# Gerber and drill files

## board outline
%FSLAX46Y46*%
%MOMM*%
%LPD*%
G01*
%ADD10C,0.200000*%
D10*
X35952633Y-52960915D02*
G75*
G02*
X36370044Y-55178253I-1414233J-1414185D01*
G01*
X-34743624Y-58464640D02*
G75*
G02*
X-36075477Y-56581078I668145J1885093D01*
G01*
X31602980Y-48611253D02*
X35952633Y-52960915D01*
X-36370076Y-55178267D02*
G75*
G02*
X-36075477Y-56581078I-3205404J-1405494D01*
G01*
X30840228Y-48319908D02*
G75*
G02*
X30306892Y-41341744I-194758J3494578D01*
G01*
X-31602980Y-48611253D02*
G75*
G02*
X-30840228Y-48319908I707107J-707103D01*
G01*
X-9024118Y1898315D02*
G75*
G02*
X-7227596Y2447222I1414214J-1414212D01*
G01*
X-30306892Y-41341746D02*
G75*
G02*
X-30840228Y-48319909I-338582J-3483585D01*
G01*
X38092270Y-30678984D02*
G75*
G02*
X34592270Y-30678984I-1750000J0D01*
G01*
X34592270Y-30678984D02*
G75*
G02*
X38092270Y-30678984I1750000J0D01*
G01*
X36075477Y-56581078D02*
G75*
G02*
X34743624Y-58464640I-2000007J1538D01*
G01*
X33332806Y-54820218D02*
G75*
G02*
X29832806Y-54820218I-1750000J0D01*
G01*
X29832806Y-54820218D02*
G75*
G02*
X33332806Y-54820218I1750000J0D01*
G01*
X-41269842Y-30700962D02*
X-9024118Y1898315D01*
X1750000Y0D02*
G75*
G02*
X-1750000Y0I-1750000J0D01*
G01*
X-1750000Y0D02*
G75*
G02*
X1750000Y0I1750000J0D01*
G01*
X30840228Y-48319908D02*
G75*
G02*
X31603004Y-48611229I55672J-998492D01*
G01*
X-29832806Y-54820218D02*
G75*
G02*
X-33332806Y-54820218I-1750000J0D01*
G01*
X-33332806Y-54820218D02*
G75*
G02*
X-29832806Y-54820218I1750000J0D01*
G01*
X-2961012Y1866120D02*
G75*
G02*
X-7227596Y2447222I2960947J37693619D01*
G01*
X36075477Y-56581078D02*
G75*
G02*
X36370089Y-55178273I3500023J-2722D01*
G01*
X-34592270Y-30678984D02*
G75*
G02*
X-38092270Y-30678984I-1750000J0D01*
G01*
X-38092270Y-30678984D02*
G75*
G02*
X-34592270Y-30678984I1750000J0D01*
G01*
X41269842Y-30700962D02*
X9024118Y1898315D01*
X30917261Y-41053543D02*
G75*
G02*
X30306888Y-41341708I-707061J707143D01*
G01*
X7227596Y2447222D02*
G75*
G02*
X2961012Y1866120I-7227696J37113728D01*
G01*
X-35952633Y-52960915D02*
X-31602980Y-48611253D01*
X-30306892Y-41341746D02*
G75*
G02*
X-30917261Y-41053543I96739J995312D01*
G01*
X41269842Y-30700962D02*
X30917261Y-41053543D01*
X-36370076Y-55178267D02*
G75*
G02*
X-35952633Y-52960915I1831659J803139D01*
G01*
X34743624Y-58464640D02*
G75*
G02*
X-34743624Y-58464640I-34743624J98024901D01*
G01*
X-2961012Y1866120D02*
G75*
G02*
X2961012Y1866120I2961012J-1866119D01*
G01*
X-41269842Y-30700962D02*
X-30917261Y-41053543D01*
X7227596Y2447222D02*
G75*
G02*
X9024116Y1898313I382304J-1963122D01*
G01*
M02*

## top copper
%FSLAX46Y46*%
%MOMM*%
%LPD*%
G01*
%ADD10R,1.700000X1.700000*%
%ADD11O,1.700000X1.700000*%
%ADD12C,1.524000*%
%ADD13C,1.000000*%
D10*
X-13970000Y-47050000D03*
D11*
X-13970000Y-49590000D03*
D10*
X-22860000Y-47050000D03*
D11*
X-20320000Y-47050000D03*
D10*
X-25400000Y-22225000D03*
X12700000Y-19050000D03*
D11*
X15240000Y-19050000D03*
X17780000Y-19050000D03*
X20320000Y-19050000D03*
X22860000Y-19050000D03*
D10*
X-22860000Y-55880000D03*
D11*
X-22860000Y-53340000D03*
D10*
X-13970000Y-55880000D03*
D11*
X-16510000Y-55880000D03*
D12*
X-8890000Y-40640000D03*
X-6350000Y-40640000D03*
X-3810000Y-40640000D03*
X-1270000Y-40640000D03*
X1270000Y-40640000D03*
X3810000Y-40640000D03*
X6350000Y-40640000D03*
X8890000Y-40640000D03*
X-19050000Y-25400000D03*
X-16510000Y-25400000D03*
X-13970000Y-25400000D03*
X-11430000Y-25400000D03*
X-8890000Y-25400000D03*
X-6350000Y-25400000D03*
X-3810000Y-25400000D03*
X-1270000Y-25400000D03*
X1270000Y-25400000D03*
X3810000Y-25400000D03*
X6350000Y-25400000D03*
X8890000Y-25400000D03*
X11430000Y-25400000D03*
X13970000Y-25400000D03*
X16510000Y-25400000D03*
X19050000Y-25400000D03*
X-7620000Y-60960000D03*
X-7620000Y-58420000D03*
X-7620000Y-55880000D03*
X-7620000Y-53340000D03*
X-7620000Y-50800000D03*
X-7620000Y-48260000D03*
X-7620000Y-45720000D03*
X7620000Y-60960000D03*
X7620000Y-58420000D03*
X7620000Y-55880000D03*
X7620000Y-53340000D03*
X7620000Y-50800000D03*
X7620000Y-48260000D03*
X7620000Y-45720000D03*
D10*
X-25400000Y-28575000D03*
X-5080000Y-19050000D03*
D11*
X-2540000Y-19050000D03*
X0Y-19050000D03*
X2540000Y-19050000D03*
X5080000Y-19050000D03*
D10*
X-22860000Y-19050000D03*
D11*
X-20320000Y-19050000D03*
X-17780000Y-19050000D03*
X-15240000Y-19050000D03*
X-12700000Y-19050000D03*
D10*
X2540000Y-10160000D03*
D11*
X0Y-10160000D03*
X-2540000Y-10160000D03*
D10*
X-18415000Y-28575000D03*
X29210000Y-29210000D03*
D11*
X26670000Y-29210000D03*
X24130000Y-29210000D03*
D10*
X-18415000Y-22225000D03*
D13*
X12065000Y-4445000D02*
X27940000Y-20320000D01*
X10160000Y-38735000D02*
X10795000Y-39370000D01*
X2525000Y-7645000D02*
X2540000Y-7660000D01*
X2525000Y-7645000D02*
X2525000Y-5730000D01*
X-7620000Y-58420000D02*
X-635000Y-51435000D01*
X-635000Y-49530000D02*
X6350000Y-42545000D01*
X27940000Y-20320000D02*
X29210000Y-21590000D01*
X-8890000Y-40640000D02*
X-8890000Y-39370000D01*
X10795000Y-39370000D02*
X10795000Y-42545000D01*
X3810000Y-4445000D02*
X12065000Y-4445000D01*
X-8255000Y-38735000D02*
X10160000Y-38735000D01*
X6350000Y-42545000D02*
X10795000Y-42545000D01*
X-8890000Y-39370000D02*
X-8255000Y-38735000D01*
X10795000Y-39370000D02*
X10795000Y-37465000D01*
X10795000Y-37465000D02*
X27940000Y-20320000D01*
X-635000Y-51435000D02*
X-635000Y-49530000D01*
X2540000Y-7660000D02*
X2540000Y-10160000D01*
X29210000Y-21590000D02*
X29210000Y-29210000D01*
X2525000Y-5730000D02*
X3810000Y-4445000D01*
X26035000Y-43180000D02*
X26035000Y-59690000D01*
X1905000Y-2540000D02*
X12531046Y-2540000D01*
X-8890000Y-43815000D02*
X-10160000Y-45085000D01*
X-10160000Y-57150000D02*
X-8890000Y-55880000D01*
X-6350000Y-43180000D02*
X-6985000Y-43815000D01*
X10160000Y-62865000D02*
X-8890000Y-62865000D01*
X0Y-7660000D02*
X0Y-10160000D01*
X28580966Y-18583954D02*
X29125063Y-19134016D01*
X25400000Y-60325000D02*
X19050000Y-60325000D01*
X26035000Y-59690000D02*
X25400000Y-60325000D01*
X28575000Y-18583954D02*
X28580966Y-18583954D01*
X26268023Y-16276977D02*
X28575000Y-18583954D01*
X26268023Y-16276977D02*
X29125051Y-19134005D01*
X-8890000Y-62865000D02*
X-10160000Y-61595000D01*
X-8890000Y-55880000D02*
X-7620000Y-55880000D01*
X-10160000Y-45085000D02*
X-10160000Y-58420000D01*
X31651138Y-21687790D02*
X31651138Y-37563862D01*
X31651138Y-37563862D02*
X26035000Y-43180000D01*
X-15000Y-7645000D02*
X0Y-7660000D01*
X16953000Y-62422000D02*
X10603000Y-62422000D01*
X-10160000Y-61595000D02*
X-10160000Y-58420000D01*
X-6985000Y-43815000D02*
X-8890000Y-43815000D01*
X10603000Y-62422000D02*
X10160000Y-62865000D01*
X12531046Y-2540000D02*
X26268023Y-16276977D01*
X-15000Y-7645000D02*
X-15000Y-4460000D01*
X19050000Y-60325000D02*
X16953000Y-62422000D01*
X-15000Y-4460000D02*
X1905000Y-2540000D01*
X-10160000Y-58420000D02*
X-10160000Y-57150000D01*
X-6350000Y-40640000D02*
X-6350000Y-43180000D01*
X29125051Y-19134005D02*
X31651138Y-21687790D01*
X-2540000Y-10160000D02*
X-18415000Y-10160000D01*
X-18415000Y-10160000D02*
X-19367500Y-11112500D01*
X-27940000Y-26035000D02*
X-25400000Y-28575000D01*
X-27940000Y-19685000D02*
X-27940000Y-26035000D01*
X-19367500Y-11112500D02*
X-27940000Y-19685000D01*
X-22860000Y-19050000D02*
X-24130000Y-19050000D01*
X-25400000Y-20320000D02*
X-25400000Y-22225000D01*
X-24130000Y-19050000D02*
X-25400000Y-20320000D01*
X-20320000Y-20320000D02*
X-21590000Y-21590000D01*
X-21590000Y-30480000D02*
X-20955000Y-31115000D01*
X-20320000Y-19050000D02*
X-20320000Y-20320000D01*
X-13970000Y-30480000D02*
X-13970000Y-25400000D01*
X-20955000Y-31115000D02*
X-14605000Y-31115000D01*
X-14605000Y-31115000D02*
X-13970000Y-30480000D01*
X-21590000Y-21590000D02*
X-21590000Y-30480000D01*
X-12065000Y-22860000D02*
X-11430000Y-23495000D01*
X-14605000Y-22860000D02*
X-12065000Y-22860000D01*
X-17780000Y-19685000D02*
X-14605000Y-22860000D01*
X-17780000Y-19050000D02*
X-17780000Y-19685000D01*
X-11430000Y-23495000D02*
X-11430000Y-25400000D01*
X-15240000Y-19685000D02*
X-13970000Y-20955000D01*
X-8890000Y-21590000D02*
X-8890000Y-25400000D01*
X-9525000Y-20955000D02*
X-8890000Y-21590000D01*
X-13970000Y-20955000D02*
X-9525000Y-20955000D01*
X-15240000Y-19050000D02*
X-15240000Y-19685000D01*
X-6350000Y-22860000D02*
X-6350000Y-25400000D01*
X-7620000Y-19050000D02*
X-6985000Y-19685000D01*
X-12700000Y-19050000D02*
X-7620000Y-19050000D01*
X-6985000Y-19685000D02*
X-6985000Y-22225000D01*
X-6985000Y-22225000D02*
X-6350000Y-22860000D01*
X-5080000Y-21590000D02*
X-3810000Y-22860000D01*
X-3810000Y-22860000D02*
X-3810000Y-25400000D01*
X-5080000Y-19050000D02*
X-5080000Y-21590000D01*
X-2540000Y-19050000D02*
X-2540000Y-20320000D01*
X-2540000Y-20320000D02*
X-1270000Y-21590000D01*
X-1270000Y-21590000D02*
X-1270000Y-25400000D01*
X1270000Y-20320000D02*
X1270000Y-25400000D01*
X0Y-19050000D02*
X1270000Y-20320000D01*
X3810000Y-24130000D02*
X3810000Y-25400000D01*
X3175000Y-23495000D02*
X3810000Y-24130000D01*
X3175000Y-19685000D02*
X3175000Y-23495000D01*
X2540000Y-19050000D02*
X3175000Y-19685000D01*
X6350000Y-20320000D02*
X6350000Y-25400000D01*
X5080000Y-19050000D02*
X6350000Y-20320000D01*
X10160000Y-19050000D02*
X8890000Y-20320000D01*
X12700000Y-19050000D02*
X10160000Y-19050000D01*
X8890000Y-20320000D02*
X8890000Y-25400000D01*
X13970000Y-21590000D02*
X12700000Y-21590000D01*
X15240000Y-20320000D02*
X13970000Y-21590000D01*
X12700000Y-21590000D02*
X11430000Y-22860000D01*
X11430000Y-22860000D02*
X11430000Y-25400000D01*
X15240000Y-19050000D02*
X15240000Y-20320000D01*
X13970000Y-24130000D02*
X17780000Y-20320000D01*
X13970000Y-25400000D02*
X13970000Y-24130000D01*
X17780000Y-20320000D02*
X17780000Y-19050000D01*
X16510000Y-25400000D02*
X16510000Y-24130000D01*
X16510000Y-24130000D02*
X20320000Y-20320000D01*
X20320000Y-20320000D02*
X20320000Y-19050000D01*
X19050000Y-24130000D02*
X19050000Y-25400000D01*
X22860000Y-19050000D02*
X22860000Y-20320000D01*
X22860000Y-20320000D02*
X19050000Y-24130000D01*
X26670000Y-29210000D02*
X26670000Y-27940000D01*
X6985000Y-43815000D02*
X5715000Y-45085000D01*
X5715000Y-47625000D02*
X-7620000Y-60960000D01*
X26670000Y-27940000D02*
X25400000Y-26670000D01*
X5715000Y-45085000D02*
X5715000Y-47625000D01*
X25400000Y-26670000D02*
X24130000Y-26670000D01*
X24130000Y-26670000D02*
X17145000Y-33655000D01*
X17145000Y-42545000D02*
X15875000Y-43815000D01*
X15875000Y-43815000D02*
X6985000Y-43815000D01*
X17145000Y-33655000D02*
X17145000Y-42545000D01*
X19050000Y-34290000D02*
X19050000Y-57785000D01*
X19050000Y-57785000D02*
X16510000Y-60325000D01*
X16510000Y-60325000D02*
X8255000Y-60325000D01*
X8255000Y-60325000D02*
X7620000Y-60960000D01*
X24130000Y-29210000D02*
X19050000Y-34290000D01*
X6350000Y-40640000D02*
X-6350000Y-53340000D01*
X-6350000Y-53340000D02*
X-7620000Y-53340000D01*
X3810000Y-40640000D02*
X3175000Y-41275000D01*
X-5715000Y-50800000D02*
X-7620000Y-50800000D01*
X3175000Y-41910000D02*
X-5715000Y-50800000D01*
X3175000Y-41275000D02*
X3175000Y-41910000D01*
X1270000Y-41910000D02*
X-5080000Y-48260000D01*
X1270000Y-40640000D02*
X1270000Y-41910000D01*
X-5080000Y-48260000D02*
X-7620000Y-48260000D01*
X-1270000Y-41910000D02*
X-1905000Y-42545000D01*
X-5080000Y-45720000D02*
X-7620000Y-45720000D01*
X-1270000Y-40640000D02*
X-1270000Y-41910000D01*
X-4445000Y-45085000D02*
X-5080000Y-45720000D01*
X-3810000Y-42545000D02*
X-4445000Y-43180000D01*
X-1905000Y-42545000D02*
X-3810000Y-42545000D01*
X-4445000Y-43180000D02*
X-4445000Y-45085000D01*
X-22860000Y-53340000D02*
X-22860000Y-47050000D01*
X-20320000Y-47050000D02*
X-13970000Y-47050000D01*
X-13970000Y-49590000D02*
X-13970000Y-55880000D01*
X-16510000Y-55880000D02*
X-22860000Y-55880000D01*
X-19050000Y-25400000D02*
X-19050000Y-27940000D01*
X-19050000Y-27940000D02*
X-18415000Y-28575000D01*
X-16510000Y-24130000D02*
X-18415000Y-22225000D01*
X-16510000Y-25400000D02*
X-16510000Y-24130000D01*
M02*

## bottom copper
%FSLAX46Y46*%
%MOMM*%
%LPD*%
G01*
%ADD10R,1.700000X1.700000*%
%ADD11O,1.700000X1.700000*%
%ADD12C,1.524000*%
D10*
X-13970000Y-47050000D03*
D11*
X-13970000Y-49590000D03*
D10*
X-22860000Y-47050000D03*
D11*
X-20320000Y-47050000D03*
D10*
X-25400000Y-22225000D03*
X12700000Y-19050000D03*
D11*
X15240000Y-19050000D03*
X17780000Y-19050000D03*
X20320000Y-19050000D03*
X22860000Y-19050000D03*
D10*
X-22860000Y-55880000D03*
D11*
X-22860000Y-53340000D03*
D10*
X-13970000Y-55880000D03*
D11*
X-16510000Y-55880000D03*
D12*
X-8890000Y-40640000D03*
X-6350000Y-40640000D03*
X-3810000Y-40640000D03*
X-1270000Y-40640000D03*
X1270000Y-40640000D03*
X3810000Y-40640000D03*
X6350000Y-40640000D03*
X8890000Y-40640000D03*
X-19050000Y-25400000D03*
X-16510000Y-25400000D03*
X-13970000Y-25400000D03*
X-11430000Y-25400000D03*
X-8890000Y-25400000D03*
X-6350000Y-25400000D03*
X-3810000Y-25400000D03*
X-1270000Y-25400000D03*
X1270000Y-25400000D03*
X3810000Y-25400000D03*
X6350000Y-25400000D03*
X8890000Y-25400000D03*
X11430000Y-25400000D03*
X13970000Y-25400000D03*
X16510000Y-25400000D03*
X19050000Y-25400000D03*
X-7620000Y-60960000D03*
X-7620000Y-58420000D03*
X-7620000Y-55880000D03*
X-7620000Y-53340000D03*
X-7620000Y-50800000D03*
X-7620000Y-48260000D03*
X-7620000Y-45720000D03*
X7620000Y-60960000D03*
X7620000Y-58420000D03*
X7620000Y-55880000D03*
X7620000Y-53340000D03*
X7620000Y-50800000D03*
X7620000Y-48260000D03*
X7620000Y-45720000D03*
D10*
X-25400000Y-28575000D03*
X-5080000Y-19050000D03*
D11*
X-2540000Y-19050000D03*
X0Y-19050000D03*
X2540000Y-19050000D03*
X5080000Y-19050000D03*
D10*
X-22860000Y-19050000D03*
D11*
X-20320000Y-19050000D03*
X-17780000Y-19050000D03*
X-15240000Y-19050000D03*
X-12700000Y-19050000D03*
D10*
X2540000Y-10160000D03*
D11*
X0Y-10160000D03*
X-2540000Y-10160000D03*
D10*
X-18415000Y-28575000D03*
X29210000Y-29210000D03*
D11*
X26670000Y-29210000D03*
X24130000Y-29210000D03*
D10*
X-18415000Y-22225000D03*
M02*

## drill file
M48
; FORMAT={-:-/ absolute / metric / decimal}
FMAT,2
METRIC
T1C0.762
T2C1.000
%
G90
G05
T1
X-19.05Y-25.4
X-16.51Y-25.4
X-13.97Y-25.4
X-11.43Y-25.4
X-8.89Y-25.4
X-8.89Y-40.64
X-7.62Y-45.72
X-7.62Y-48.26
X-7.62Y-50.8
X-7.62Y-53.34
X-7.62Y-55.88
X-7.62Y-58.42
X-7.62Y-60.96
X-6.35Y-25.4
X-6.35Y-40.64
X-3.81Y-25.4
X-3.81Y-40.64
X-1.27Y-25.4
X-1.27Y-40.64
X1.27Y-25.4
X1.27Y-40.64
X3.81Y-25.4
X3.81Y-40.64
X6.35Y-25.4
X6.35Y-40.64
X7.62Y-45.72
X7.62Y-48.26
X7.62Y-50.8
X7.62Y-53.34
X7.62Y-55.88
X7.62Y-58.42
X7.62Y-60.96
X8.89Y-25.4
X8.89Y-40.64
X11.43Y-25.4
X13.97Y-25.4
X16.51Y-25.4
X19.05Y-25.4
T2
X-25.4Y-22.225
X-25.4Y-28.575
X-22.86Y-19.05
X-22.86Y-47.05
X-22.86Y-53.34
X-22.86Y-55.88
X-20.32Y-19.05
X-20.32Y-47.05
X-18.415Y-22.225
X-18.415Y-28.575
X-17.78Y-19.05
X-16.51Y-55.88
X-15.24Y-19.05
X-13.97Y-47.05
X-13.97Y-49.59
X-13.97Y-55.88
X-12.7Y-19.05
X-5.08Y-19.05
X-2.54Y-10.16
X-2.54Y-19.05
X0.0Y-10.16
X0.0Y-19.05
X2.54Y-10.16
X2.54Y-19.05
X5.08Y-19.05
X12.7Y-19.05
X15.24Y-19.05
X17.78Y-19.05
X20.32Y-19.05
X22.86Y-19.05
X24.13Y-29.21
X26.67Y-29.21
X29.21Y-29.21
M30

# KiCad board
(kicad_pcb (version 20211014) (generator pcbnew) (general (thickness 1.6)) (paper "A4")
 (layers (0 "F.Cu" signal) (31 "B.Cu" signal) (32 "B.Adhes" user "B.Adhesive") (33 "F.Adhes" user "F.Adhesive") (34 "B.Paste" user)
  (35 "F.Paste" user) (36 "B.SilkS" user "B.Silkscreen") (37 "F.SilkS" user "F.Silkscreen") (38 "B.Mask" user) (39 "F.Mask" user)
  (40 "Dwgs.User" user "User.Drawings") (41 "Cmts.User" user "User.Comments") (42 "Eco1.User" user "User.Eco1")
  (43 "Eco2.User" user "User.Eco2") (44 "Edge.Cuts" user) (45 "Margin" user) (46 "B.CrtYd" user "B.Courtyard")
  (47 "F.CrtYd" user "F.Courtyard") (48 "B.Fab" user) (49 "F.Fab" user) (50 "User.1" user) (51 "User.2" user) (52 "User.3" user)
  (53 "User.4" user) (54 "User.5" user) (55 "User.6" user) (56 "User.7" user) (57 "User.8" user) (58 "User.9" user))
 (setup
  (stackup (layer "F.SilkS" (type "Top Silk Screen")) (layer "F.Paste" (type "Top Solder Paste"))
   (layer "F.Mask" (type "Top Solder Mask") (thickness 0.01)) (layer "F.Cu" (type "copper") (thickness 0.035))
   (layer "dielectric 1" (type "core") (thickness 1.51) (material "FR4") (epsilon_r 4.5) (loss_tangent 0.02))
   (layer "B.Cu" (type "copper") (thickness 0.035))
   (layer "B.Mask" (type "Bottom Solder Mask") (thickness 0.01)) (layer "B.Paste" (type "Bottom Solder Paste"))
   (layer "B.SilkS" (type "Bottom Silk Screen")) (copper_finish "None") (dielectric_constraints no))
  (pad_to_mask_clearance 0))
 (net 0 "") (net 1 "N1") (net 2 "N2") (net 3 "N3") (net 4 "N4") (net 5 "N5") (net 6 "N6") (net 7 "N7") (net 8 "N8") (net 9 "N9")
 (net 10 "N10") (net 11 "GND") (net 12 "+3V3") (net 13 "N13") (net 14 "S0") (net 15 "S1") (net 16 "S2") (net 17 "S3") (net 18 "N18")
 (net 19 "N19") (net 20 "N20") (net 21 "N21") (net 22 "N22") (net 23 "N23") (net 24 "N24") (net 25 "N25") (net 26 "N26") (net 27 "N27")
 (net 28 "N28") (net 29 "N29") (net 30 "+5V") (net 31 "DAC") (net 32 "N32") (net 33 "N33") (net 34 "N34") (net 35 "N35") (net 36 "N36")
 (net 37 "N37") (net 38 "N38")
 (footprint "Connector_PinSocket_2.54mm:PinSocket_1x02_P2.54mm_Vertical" (layer "F.Cu") (at -13.97 47.05)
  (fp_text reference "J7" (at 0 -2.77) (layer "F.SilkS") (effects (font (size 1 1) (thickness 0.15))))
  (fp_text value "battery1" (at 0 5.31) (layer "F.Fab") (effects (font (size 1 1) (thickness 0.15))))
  (pad "1" thru_hole rect (at 0 0) (size 1.7 1.7) (drill 1) (layers *.Cu *.Mask) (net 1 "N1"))
  (pad "2" thru_hole oval (at 0 2.54) (size 1.7 1.7) (drill 1) (layers *.Cu *.Mask) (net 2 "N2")))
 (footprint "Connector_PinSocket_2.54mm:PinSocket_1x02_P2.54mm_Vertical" (layer "F.Cu") (at -22.86 47.05 90)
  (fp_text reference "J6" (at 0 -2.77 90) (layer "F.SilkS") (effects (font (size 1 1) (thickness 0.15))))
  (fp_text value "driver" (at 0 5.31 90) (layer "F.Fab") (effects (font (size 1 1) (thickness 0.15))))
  (pad "1" thru_hole rect (at 0 0 90) (size 1.7 1.7) (drill 1) (layers *.Cu *.Mask) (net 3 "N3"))
  (pad "2" thru_hole oval (at 0 2.54 90) (size 1.7 1.7) (drill 1) (layers *.Cu *.Mask) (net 1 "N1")))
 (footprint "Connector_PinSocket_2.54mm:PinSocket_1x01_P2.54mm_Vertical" (layer "F.Cu") (at -25.4 22.225)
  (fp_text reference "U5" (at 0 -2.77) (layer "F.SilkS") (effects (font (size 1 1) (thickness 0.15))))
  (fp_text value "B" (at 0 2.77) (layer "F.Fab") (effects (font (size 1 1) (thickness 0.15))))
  (pad "1" thru_hole rect (at 0 0) (size 1.7 1.7) (drill 1) (layers *.Cu *.Mask) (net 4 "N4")))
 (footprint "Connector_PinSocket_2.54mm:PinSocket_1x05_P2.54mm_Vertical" (layer "F.Cu") (at 12.7 19.05 90)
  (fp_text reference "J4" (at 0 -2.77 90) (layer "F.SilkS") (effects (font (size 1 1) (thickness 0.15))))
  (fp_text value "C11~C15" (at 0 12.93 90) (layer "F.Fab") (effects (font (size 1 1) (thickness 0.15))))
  (pad "1" thru_hole rect (at 0 0 90) (size 1.7 1.7) (drill 1) (layers *.Cu *.Mask) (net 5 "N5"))
  (pad "2" thru_hole oval (at 0 2.54 90) (size 1.7 1.7) (drill 1) (layers *.Cu *.Mask) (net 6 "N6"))
  (pad "3" thru_hole oval (at 0 5.08 90) (size 1.7 1.7) (drill 1) (layers *.Cu *.Mask) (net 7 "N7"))
  (pad "4" thru_hole oval (at 0 7.62 90) (size 1.7 1.7) (drill 1) (layers *.Cu *.Mask) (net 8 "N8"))
  (pad "5" thru_hole oval (at 0 10.16 90) (size 1.7 1.7) (drill 1) (layers *.Cu *.Mask) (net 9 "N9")))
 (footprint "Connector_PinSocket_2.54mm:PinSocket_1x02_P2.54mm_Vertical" (layer "F.Cu") (at -22.86 55.88 180)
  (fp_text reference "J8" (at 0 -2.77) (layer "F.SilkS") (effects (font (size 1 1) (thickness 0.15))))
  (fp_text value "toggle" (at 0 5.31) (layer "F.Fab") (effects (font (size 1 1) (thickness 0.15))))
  (pad "1" thru_hole rect (at 0 0 180) (size 1.7 1.7) (drill 1) (layers *.Cu *.Mask) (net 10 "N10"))
  (pad "2" thru_hole oval (at 0 2.54 180) (size 1.7 1.7) (drill 1) (layers *.Cu *.Mask) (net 3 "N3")))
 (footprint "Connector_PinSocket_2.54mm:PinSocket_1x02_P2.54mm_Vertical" (layer "F.Cu") (at -13.97 55.88 -90)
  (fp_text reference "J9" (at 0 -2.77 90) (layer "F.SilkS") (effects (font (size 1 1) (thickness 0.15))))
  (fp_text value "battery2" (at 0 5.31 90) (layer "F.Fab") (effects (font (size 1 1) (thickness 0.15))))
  (pad "1" thru_hole rect (at 0 0 270) (size 1.7 1.7) (drill 1) (layers *.Cu *.Mask) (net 2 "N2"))
  (pad "2" thru_hole oval (at 0 2.54 270) (size 1.7 1.7) (drill 1) (layers *.Cu *.Mask) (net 10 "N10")))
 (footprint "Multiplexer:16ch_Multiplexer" (layer "F.Cu") (at -1.27 25.4)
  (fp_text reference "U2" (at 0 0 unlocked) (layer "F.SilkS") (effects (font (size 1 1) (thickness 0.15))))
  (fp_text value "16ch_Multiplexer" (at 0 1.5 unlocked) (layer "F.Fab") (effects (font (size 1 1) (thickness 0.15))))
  (pad "1" thru_hole circle (at -7.62 15.24) (size 1.524 1.524) (drill 0.762) (layers *.Cu *.Mask) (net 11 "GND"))
  (pad "2" thru_hole circle (at -5.08 15.24) (size 1.524 1.524) (drill 0.762) (layers *.Cu *.Mask) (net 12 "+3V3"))
  (pad "3" thru_hole circle (at -2.54 15.24) (size 1.524 1.524) (drill 0.762) (layers *.Cu *.Mask) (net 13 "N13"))
  (pad "4" thru_hole circle (at 0 15.24) (size 1.524 1.524) (drill 0.762) (layers *.Cu *.Mask) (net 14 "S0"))
  (pad "5" thru_hole circle (at 2.54 15.24) (size 1.524 1.524) (drill 0.762) (layers *.Cu *.Mask) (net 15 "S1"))
  (pad "6" thru_hole circle (at 5.08 15.24) (size 1.524 1.524) (drill 0.762) (layers *.Cu *.Mask) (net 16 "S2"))
  (pad "7" thru_hole circle (at 7.62 15.24) (size 1.524 1.524) (drill 0.762) (layers *.Cu *.Mask) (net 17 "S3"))
  (pad "8" thru_hole circle (at 10.16 15.24) (size 1.524 1.524) (drill 0.762) (layers *.Cu *.Mask) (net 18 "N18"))
  (pad "9" thru_hole circle (at -17.78 0) (size 1.524 1.524) (drill 0.762) (layers *.Cu *.Mask) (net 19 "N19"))
  (pad "10" thru_hole circle (at -15.24 0) (size 1.524 1.524) (drill 0.762) (layers *.Cu *.Mask) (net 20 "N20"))
  (pad "11" thru_hole circle (at -12.7 0) (size 1.524 1.524) (drill 0.762) (layers *.Cu *.Mask) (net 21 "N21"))
  (pad "12" thru_hole circle (at -10.16 0) (size 1.524 1.524) (drill 0.762) (layers *.Cu *.Mask) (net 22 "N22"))
  (pad "13" thru_hole circle (at -7.62 0) (size 1.524 1.524) (drill 0.762) (layers *.Cu *.Mask) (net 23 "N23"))
  (pad "14" thru_hole circle (at -5.08 0) (size 1.524 1.524) (drill 0.762) (layers *.Cu *.Mask) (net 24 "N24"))
  (pad "15" thru_hole circle (at -2.54 0) (size 1.524 1.524) (drill 0.762) (layers *.Cu *.Mask) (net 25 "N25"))
  (pad "16" thru_hole circle (at 0 0) (size 1.524 1.524) (drill 0.762) (layers *.Cu *.Mask) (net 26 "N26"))
  (pad "17" thru_hole circle (at 2.54 0) (size 1.524 1.524) (drill 0.762) (layers *.Cu *.Mask) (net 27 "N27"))
  (pad "18" thru_hole circle (at 5.08 0) (size 1.524 1.524) (drill 0.762) (layers *.Cu *.Mask) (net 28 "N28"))
  (pad "19" thru_hole circle (at 7.62 0) (size 1.524 1.524) (drill 0.762) (layers *.Cu *.Mask) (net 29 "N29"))
  (pad "20" thru_hole circle (at 10.16 0) (size 1.524 1.524) (drill 0.762) (layers *.Cu *.Mask) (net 5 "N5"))
  (pad "21" thru_hole circle (at 12.7 0) (size 1.524 1.524) (drill 0.762) (layers *.Cu *.Mask) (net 6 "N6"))
  (pad "22" thru_hole circle (at 15.24 0) (size 1.524 1.524) (drill 0.762) (layers *.Cu *.Mask) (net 7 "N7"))
  (pad "23" thru_hole circle (at 17.78 0) (size 1.524 1.524) (drill 0.762) (layers *.Cu *.Mask) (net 8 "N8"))
  (pad "24" thru_hole circle (at 20.32 0) (size 1.524 1.524) (drill 0.762) (layers *.Cu *.Mask) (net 9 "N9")))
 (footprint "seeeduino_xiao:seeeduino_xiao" (layer "F.Cu") (at 0 63.5 180)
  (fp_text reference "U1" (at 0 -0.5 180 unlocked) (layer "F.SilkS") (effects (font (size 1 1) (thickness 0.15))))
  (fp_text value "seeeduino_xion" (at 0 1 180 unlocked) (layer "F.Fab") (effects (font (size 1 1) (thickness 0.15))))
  (pad "1" thru_hole circle (at 7.62 2.54 180) (size 1.524 1.524) (drill 0.762) (layers *.Cu *.Mask) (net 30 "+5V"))
  (pad "2" thru_hole circle (at 7.62 5.08 180) (size 1.524 1.524) (drill 0.762) (layers *.Cu *.Mask) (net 11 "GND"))
  (pad "3" thru_hole circle (at 7.62 7.62 180) (size 1.524 1.524) (drill 0.762) (layers *.Cu *.Mask) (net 12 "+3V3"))
  (pad "4" thru_hole circle (at 7.62 10.16 180) (size 1.524 1.524) (drill 0.762) (layers *.Cu *.Mask) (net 17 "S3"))
  (pad "5" thru_hole circle (at 7.62 12.7 180) (size 1.524 1.524) (drill 0.762) (layers *.Cu *.Mask) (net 16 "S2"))
  (pad "6" thru_hole circle (at 7.62 15.24 180) (size 1.524 1.524) (drill 0.762) (layers *.Cu *.Mask) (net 15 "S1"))
  (pad "7" thru_hole circle (at 7.62 17.78 180) (size 1.524 1.524) (drill 0.762) (layers *.Cu *.Mask) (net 14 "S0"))
  (pad "8" thru_hole circle (at -7.62 2.54 180) (size 1.524 1.524) (drill 0.762) (layers *.Cu *.Mask) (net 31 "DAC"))
  (pad "9" thru_hole circle (at -7.62 5.08 180) (size 1.524 1.524) (drill 0.762) (layers *.Cu *.Mask) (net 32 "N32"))
  (pad "10" thru_hole circle (at -7.62 7.62 180) (size 1.524 1.524) (drill 0.762) (layers *.Cu *.Mask) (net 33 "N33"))
  (pad "11" thru_hole circle (at -7.62 10.16 180) (size 1.524 1.524) (drill 0.762) (layers *.Cu *.Mask) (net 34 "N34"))
  (pad "12" thru_hole circle (at -7.62 12.7 180) (size 1.524 1.524) (drill 0.762) (layers *.Cu *.Mask) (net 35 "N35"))
  (pad "13" thru_hole circle (at -7.62 15.24 180) (size 1.524 1.524) (drill 0.762) (layers *.Cu *.Mask) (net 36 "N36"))
  (pad "14" thru_hole circle (at -7.62 17.78 180) (size 1.524 1.524) (drill 0.762) (layers *.Cu *.Mask) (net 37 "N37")))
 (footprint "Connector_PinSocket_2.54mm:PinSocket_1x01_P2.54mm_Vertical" (layer "F.Cu") (at -25.4 28.575)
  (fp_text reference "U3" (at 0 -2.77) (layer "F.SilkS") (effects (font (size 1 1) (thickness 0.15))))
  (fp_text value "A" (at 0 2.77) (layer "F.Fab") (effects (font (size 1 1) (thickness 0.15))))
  (pad "1" thru_hole rect (at 0 0) (size 1.7 1.7) (drill 1) (layers *.Cu *.Mask) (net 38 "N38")))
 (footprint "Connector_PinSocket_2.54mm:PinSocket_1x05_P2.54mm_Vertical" (layer "F.Cu") (at -5.08 19.05 90)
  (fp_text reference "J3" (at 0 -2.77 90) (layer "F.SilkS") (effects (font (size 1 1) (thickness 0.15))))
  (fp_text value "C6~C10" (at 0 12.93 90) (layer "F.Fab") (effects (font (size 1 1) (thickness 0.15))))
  (pad "1" thru_hole rect (at 0 0 90) (size 1.7 1.7) (drill 1) (layers *.Cu *.Mask) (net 25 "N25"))
  (pad "2" thru_hole oval (at 0 2.54 90) (size 1.7 1.7) (drill 1) (layers *.Cu *.Mask) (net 26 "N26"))
  (pad "3" thru_hole oval (at 0 5.08 90) (size 1.7 1.7) (drill 1) (layers *.Cu *.Mask) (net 27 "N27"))
  (pad "4" thru_hole oval (at 0 7.62 90) (size 1.7 1.7) (drill 1) (layers *.Cu *.Mask) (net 28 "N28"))
  (pad "5" thru_hole oval (at 0 10.16 90) (size 1.7 1.7) (drill 1) (layers *.Cu *.Mask) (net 29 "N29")))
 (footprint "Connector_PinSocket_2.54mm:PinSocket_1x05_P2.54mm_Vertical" (layer "F.Cu") (at -22.86 19.05 90)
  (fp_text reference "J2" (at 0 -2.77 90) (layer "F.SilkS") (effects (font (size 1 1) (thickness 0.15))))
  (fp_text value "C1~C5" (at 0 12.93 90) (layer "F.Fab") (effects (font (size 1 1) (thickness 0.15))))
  (pad "1" thru_hole rect (at 0 0 90) (size 1.7 1.7) (drill 1) (layers *.Cu *.Mask) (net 4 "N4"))
  (pad "2" thru_hole oval (at 0 2.54 90) (size 1.7 1.7) (drill 1) (layers *.Cu *.Mask) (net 21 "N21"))
  (pad "3" thru_hole oval (at 0 5.08 90) (size 1.7 1.7) (drill 1) (layers *.Cu *.Mask) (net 22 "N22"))
  (pad "4" thru_hole oval (at 0 7.62 90) (size 1.7 1.7) (drill 1) (layers *.Cu *.Mask) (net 23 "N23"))
  (pad "5" thru_hole oval (at 0 10.16 90) (size 1.7 1.7) (drill 1) (layers *.Cu *.Mask) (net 24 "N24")))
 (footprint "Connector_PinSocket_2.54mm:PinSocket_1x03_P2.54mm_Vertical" (layer "F.Cu") (at 2.54 10.16 -90)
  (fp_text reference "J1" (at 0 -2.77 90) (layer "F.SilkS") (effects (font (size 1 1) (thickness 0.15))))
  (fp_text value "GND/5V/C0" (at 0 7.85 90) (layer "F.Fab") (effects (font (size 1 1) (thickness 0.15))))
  (pad "1" thru_hole rect (at 0 0 270) (size 1.7 1.7) (drill 1) (layers *.Cu *.Mask) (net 11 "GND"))
  (pad "2" thru_hole oval (at 0 2.54 270) (size 1.7 1.7) (drill 1) (layers *.Cu *.Mask) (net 12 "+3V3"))
  (pad "3" thru_hole oval (at 0 5.08 270) (size 1.7 1.7) (drill 1) (layers *.Cu *.Mask) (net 38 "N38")))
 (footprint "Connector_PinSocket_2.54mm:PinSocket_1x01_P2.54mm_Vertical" (layer "F.Cu") (at -18.415 28.575)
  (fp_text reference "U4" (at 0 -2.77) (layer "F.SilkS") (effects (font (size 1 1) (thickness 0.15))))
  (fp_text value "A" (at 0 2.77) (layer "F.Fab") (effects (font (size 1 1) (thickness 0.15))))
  (pad "1" thru_hole rect (at 0 0) (size 1.7 1.7) (drill 1) (layers *.Cu *.Mask) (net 19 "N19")))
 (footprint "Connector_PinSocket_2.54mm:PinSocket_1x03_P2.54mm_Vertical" (layer "F.Cu") (at 29.21 29.21 -90)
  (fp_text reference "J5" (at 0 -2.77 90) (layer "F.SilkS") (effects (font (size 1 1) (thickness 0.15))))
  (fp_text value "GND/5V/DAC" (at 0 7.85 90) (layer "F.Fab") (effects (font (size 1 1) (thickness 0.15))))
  (pad "1" thru_hole rect (at 0 0 270) (size 1.7 1.7) (drill 1) (layers *.Cu *.Mask) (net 11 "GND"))
  (pad "2" thru_hole oval (at 0 2.54 270) (size 1.7 1.7) (drill 1) (layers *.Cu *.Mask) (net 30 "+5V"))
  (pad "3" thru_hole oval (at 0 5.08 270) (size 1.7 1.7) (drill 1) (layers *.Cu *.Mask) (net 31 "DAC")))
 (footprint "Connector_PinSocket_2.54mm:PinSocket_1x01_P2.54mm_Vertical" (layer "F.Cu") (at -18.415 22.225)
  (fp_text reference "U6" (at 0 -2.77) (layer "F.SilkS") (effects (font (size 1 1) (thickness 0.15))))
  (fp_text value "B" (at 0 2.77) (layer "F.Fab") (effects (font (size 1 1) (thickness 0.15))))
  (pad "1" thru_hole rect (at 0 0) (size 1.7 1.7) (drill 1) (layers *.Cu *.Mask) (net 20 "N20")))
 (gr_arc (start 35.952633 52.960915) (mid 36.503891 54.005104) (end 36.370076 55.178267) (layer "Edge.Cuts") (width 0.2))
 (gr_arc (start -34.743624 58.46464) (mid -35.708482 57.734231) (end -36.075477 56.581078) (layer "Edge.Cuts") (width 0.2))
 (gr_line (start 31.60298 48.611253) (end 35.952633 52.960915) (layer "Edge.Cuts") (width 0.2))
 (gr_arc (start -36.370076 55.178267) (mid -36.150193 55.86443) (end -36.075477 56.581078) (layer "Edge.Cuts") (width 0.2))
 (gr_arc (start 30.840228 48.319908) (mid 27.155652 45.092056) (end 30.306892 41.341746) (layer "Edge.Cuts") (width 0.2))
 (gr_arc (start -31.60298 48.611253) (mid -31.252694 48.384186) (end -30.840228 48.319908) (layer "Edge.Cuts") (width 0.2))
 (gr_arc (start -9.024118 -1.898315) (mid -8.194312 -2.396814) (end -7.227596 -2.447222) (layer "Edge.Cuts") (width 0.2))
 (gr_arc (start -30.306892 41.341746) (mid -27.155652 45.092056) (end -30.840228 48.319908) (layer "Edge.Cuts") (width 0.2))
 (gr_circle (center 36.34227 30.678984) (end 36.34227 28.928984) (layer "Edge.Cuts") (width 0.2) (fill none))
 (gr_arc (start 36.075477 56.581078) (mid 35.708481 57.73423) (end 34.743624 58.46464) (layer "Edge.Cuts") (width 0.2))
 (gr_circle (center 31.582806 54.820218) (end 31.582806 53.070218) (layer "Edge.Cuts") (width 0.2) (fill none))
 (gr_line (start -41.269842 30.700962) (end -9.024118 -1.898315) (layer "Edge.Cuts") (width 0.2))
 (gr_circle (center 0 0) (end 0 -1.75) (layer "Edge.Cuts") (width 0.2) (fill none))
 (gr_arc (start 30.840228 48.319908) (mid 31.252694 48.384186) (end 31.60298 48.611253) (layer "Edge.Cuts") (width 0.2))
 (gr_circle (center -31.582806 54.820218) (end -31.582806 53.070218) (layer "Edge.Cuts") (width 0.2) (fill none))
 (gr_arc (start -2.961012 -1.86612) (mid -5.102583 -2.095884) (end -7.227596 -2.447222) (layer "Edge.Cuts") (width 0.2))
 (gr_arc (start 36.075477 56.581078) (mid 36.150193 55.86443) (end 36.370076 55.178267) (layer "Edge.Cuts") (width 0.2))
 (gr_circle (center -36.34227 30.678984) (end -36.34227 28.928984) (layer "Edge.Cuts") (width 0.2) (fill none))
 (gr_line (start 41.269842 30.700962) (end 9.024118 -1.898315) (layer "Edge.Cuts") (width 0.2))
 (gr_arc (start 30.917261 41.053543) (mid 30.637128 41.250701) (end 30.306892 41.341746) (layer "Edge.Cuts") (width 0.2))
 (gr_arc (start 7.227596 -2.447222) (mid 5.102583 -2.095886) (end 2.961012 -1.86612) (layer "Edge.Cuts") (width 0.2))
 (gr_line (start -35.952633 52.960915) (end -31.60298 48.611253) (layer "Edge.Cuts") (width 0.2))
 (gr_arc (start -30.306892 41.341746) (mid -30.637128 41.2507) (end -30.917261 41.053543) (layer "Edge.Cuts") (width 0.2))
 (gr_line (start 41.269842 30.700962) (end 30.917261 41.053543) (layer "Edge.Cuts") (width 0.2))
 (gr_arc (start -36.370076 55.178267) (mid -36.503891 54.005104) (end -35.952633 52.960915) (layer "Edge.Cuts") (width 0.2))
 (gr_arc (start 34.743624 58.46464) (mid 0 64.439742) (end -34.743624 58.46464) (layer "Edge.Cuts") (width 0.2))
 (gr_arc (start -2.961012 -1.86612) (mid 0 -3.5) (end 2.961012 -1.86612) (layer "Edge.Cuts") (width 0.2))
 (gr_line (start -41.269842 30.700962) (end -30.917261 41.053543) (layer "Edge.Cuts") (width 0.2))
 (gr_arc (start 7.227596 -2.447222) (mid 8.194312 -2.396814) (end 9.024118 -1.898315) (layer "Edge.Cuts") (width 0.2))
 (segment (start 12.065 4.445) (end 27.94 20.32) (width 1) (layer "F.Cu") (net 11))
 (segment (start 10.16 38.735) (end 10.795 39.37) (width 1) (layer "F.Cu") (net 11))
 (segment (start 2.525 7.645) (end 2.54 7.66) (width 1) (layer "F.Cu") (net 11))
 (segment (start 2.525 7.645) (end 2.525 5.73) (width 1) (layer "F.Cu") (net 11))
 (segment (start -7.62 58.42) (end -0.635 51.435) (width 1) (layer "F.Cu") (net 11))
 (segment (start -0.635 49.53) (end 6.35 42.545) (width 1) (layer "F.Cu") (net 11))
 (segment (start 27.94 20.32) (end 29.21 21.59) (width 1) (layer "F.Cu") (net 11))
 (segment (start -8.89 40.64) (end -8.89 39.37) (width 1) (layer "F.Cu") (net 11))
 (segment (start 10.795 39.37) (end 10.795 42.545) (width 1) (layer "F.Cu") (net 11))
 (segment (start 3.81 4.445) (end 12.065 4.445) (width 1) (layer "F.Cu") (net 11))
 (segment (start -8.255 38.735) (end 10.16 38.735) (width 1) (layer "F.Cu") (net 11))
 (segment (start 6.35 42.545) (end 10.795 42.545) (width 1) (layer "F.Cu") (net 11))
 (segment (start -8.89 39.37) (end -8.255 38.735) (width 1) (layer "F.Cu") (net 11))
 (segment (start 10.795 39.37) (end 10.795 37.465) (width 1) (layer "F.Cu") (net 11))
 (segment (start 10.795 37.465) (end 27.94 20.32) (width 1) (layer "F.Cu") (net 11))
 (segment (start -0.635 51.435) (end -0.635 49.53) (width 1) (layer "F.Cu") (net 11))
 (segment (start 2.54 7.66) (end 2.54 10.16) (width 1) (layer "F.Cu") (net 11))
 (segment (start 29.21 21.59) (end 29.21 29.21) (width 1) (layer "F.Cu") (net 11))
 (segment (start 2.525 5.73) (end 3.81 4.445) (width 1) (layer "F.Cu") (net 11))
 (segment (start 26.035 43.18) (end 26.035 59.69) (width 1) (layer "F.Cu") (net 12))
 (segment (start 1.905 2.54) (end 12.531046 2.54) (width 1) (layer "F.Cu") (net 12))
 (segment (start -8.89 43.815) (end -10.16 45.085) (width 1) (layer "F.Cu") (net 12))
 (segment (start -10.16 57.15) (end -8.89 55.88) (width 1) (layer "F.Cu") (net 12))
 (segment (start -6.35 43.18) (end -6.985 43.815) (width 1) (layer "F.Cu") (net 12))
 (segment (start 10.16 62.865) (end -8.89 62.865) (width 1) (layer "F.Cu") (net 12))
 (segment (start 0 7.66) (end 0 10.16) (width 1) (layer "F.Cu") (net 12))
 (segment (start 28.580966 18.583954) (end 29.125063 19.134016) (width 1) (layer "F.Cu") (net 12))
 (segment (start 25.4 60.325) (end 19.05 60.325) (width 1) (layer "F.Cu") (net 12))
 (segment (start 26.035 59.69) (end 25.4 60.325) (width 1) (layer "F.Cu") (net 12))
 (segment (start 28.575 18.583954) (end 28.580966 18.583954) (width 1) (layer "F.Cu") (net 12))
 (segment (start 26.268023 16.276977) (end 28.575 18.583954) (width 1) (layer "F.Cu") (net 12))
 (segment (start 26.268023 16.276977) (end 29.125051 19.134005) (width 1) (layer "F.Cu") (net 12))
 (segment (start -8.89 62.865) (end -10.16 61.595) (width 1) (layer "F.Cu") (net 12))
 (segment (start -8.89 55.88) (end -7.62 55.88) (width 1) (layer "F.Cu") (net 12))
 (segment (start -10.16 45.085) (end -10.16 58.42) (width 1) (layer "F.Cu") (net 12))
 (segment (start 31.651138 21.68779) (end 31.651138 37.563862) (width 1) (layer "F.Cu") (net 12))
 (segment (start 31.651138 37.563862) (end 26.035 43.18) (width 1) (layer "F.Cu") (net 12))
 (segment (start -0.015 7.645) (end 0 7.66) (width 1) (layer "F.Cu") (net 12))
 (segment (start 16.953 62.422) (end 10.603 62.422) (width 1) (layer "F.Cu") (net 12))
 (segment (start -10.16 61.595) (end -10.16 58.42) (width 1) (layer "F.Cu") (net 12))
 (segment (start -6.985 43.815) (end -8.89 43.815) (width 1) (layer "F.Cu") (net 12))
 (segment (start 10.603 62.422) (end 10.16 62.865) (width 1) (layer "F.Cu") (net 12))
 (segment (start 12.531046 2.54) (end 26.268023 16.276977) (width 1) (layer "F.Cu") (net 12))
 (segment (start -0.015 7.645) (end -0.015 4.46) (width 1) (layer "F.Cu") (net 12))
 (segment (start 19.05 60.325) (end 16.953 62.422) (width 1) (layer "F.Cu") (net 12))
 (segment (start -0.015 4.46) (end 1.905 2.54) (width 1) (layer "F.Cu") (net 12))
 (segment (start -10.16 58.42) (end -10.16 57.15) (width 1) (layer "F.Cu") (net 12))
 (segment (start -6.35 40.64) (end -6.35 43.18) (width 1) (layer "F.Cu") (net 12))
 (segment (start 29.125051 19.134005) (end 31.651138 21.68779) (width 1) (layer "F.Cu") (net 12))
 (segment (start -2.54 10.16) (end -18.415 10.16) (width 1) (layer "F.Cu") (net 38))
 (segment (start -18.415 10.16) (end -19.3675 11.1125) (width 1) (layer "F.Cu") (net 38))
 (segment (start -27.94 26.035) (end -25.4 28.575) (width 1) (layer "F.Cu") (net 38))
 (segment (start -27.94 19.685) (end -27.94 26.035) (width 1) (layer "F.Cu") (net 38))
 (segment (start -19.3675 11.1125) (end -27.94 19.685) (width 1) (layer "F.Cu") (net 38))
 (segment (start -22.86 19.05) (end -24.13 19.05) (width 1) (layer "F.Cu") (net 4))
 (segment (start -25.4 20.32) (end -25.4 22.225) (width 1) (layer "F.Cu") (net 4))
 (segment (start -24.13 19.05) (end -25.4 20.32) (width 1) (layer "F.Cu") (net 4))
 (segment (start -20.32 20.32) (end -21.59 21.59) (width 1) (layer "F.Cu") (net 21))
 (segment (start -21.59 30.48) (end -20.955 31.115) (width 1) (layer "F.Cu") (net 21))
 (segment (start -20.32 19.05) (end -20.32 20.32) (width 1) (layer "F.Cu") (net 21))
 (segment (start -13.97 30.48) (end -13.97 25.4) (width 1) (layer "F.Cu") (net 21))
 (segment (start -20.955 31.115) (end -14.605 31.115) (width 1) (layer "F.Cu") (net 21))
 (segment (start -14.605 31.115) (end -13.97 30.48) (width 1) (layer "F.Cu") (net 21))
 (segment (start -21.59 21.59) (end -21.59 30.48) (width 1) (layer "F.Cu") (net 21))
 (segment (start -12.065 22.86) (end -11.43 23.495) (width 1) (layer "F.Cu") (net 22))
 (segment (start -14.605 22.86) (end -12.065 22.86) (width 1) (layer "F.Cu") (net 22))
 (segment (start -17.78 19.685) (end -14.605 22.86) (width 1) (layer "F.Cu") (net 22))
 (segment (start -17.78 19.05) (end -17.78 19.685) (width 1) (layer "F.Cu") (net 22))
 (segment (start -11.43 23.495) (end -11.43 25.4) (width 1) (layer "F.Cu") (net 22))
 (segment (start -15.24 19.685) (end -13.97 20.955) (width 1) (layer "F.Cu") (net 23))
 (segment (start -8.89 21.59) (end -8.89 25.4) (width 1) (layer "F.Cu") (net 23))
 (segment (start -9.525 20.955) (end -8.89 21.59) (width 1) (layer "F.Cu") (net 23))
 (segment (start -13.97 20.955) (end -9.525 20.955) (width 1) (layer "F.Cu") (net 23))
 (segment (start -15.24 19.05) (end -15.24 19.685) (width 1) (layer "F.Cu") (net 23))
 (segment (start -6.35 22.86) (end -6.35 25.4) (width 1) (layer "F.Cu") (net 24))
 (segment (start -7.62 19.05) (end -6.985 19.685) (width 1) (layer "F.Cu") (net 24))
 (segment (start -12.7 19.05) (end -7.62 19.05) (width 1) (layer "F.Cu") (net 24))
 (segment (start -6.985 19.685) (end -6.985 22.225) (width 1) (layer "F.Cu") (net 24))
 (segment (start -6.985 22.225) (end -6.35 22.86) (width 1) (layer "F.Cu") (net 24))
 (segment (start -5.08 21.59) (end -3.81 22.86) (width 1) (layer "F.Cu") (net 25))
 (segment (start -3.81 22.86) (end -3.81 25.4) (width 1) (layer "F.Cu") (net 25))
 (segment (start -5.08 19.05) (end -5.08 21.59) (width 1) (layer "F.Cu") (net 25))
 (segment (start -2.54 19.05) (end -2.54 20.32) (width 1) (layer "F.Cu") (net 26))
 (segment (start -2.54 20.32) (end -1.27 21.59) (width 1) (layer "F.Cu") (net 26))
 (segment (start -1.27 21.59) (end -1.27 25.4) (width 1) (layer "F.Cu") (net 26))
 (segment (start 1.27 20.32) (end 1.27 25.4) (width 1) (layer "F.Cu") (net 27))
 (segment (start 0 19.05) (end 1.27 20.32) (width 1) (layer "F.Cu") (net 27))
 (segment (start 3.81 24.13) (end 3.81 25.4) (width 1) (layer "F.Cu") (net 28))
 (segment (start 3.175 23.495) (end 3.81 24.13) (width 1) (layer "F.Cu") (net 28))
 (segment (start 3.175 19.685) (end 3.175 23.495) (width 1) (layer "F.Cu") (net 28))
 (segment (start 2.54 19.05) (end 3.175 19.685) (width 1) (layer "F.Cu") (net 28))
 (segment (start 6.35 20.32) (end 6.35 25.4) (width 1) (layer "F.Cu") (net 29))
 (segment (start 5.08 19.05) (end 6.35 20.32) (width 1) (layer "F.Cu") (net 29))
 (segment (start 10.16 19.05) (end 8.89 20.32) (width 1) (layer "F.Cu") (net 5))
 (segment (start 12.7 19.05) (end 10.16 19.05) (width 1) (layer "F.Cu") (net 5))
 (segment (start 8.89 20.32) (end 8.89 25.4) (width 1) (layer "F.Cu") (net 5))
 (segment (start 13.97 21.59) (end 12.7 21.59) (width 1) (layer "F.Cu") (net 6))
 (segment (start 15.24 20.32) (end 13.97 21.59) (width 1) (layer "F.Cu") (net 6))
 (segment (start 12.7 21.59) (end 11.43 22.86) (width 1) (layer "F.Cu") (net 6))
 (segment (start 11.43 22.86) (end 11.43 25.4) (width 1) (layer "F.Cu") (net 6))
 (segment (start 15.24 19.05) (end 15.24 20.32) (width 1) (layer "F.Cu") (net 6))
 (segment (start 13.97 24.13) (end 17.78 20.32) (width 1) (layer "F.Cu") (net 7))
 (segment (start 13.97 25.4) (end 13.97 24.13) (width 1) (layer "F.Cu") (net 7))
 (segment (start 17.78 20.32) (end 17.78 19.05) (width 1) (layer "F.Cu") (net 7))
 (segment (start 16.51 25.4) (end 16.51 24.13) (width 1) (layer "F.Cu") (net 8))
 (segment (start 16.51 24.13) (end 20.32 20.32) (width 1) (layer "F.Cu") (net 8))
 (segment (start 20.32 20.32) (end 20.32 19.05) (width 1) (layer "F.Cu") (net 8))
 (segment (start 19.05 24.13) (end 19.05 25.4) (width 1) (layer "F.Cu") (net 9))
 (segment (start 22.86 19.05) (end 22.86 20.32) (width 1) (layer "F.Cu") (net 9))
 (segment (start 22.86 20.32) (end 19.05 24.13) (width 1) (layer "F.Cu") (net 9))
 (segment (start 26.67 29.21) (end 26.67 27.94) (width 1) (layer "F.Cu") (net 30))
 (segment (start 6.985 43.815) (end 5.715 45.085) (width 1) (layer "F.Cu") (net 30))
 (segment (start 5.715 47.625) (end -7.62 60.96) (width 1) (layer "F.Cu") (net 30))
 (segment (start 26.67 27.94) (end 25.4 26.67) (width 1) (layer "F.Cu") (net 30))
 (segment (start 5.715 45.085) (end 5.715 47.625) (width 1) (layer "F.Cu") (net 30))
 (segment (start 25.4 26.67) (end 24.13 26.67) (width 1) (layer "F.Cu") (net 30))
 (segment (start 24.13 26.67) (end 17.145 33.655) (width 1) (layer "F.Cu") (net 30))
 (segment (start 17.145 42.545) (end 15.875 43.815) (width 1) (layer "F.Cu") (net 30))
 (segment (start 15.875 43.815) (end 6.985 43.815) (width 1) (layer "F.Cu") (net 30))
 (segment (start 17.145 33.655) (end 17.145 42.545) (width 1) (layer "F.Cu") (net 30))
 (segment (start 19.05 34.29) (end 19.05 57.785) (width 1) (layer "F.Cu") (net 31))
 (segment (start 19.05 57.785) (end 16.51 60.325) (width 1) (layer "F.Cu") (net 31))
 (segment (start 16.51 60.325) (end 8.255 60.325) (width 1) (layer "F.Cu") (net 31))
 (segment (start 8.255 60.325) (end 7.62 60.96) (width 1) (layer "F.Cu") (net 31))
 (segment (start 24.13 29.21) (end 19.05 34.29) (width 1) (layer "F.Cu") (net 31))
 (segment (start 6.35 40.64) (end -6.35 53.34) (width 1) (layer "F.Cu") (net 17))
 (segment (start -6.35 53.34) (end -7.62 53.34) (width 1) (layer "F.Cu") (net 17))
 (segment (start 3.81 40.64) (end 3.175 41.275) (width 1) (layer "F.Cu") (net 16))
 (segment (start -5.715 50.8) (end -7.62 50.8) (width 1) (layer "F.Cu") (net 16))
 (segment (start 3.175 41.91) (end -5.715 50.8) (width 1) (layer "F.Cu") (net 16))
 (segment (start 3.175 41.275) (end 3.175 41.91) (width 1) (layer "F.Cu") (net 16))
 (segment (start 1.27 41.91) (end -5.08 48.26) (width 1) (layer "F.Cu") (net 15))
 (segment (start 1.27 40.64) (end 1.27 41.91) (width 1) (layer "F.Cu") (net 15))
 (segment (start -5.08 48.26) (end -7.62 48.26) (width 1) (layer "F.Cu") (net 15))
 (segment (start -1.27 41.91) (end -1.905 42.545) (width 1) (layer "F.Cu") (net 14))
 (segment (start -5.08 45.72) (end -7.62 45.72) (width 1) (layer "F.Cu") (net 14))
 (segment (start -1.27 40.64) (end -1.27 41.91) (width 1) (layer "F.Cu") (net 14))
 (segment (start -4.445 45.085) (end -5.08 45.72) (width 1) (layer "F.Cu") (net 14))
 (segment (start -3.81 42.545) (end -4.445 43.18) (width 1) (layer "F.Cu") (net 14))
 (segment (start -1.905 42.545) (end -3.81 42.545) (width 1) (layer "F.Cu") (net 14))
 (segment (start -4.445 43.18) (end -4.445 45.085) (width 1) (layer "F.Cu") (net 14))
 (segment (start -22.86 53.34) (end -22.86 47.05) (width 1) (layer "F.Cu") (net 3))
 (segment (start -20.32 47.05) (end -13.97 47.05) (width 1) (layer "F.Cu") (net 1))
 (segment (start -13.97 49.59) (end -13.97 55.88) (width 1) (layer "F.Cu") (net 2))
 (segment (start -16.51 55.88) (end -22.86 55.88) (width 1) (layer "F.Cu") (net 10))
 (segment (start -19.05 25.4) (end -19.05 27.94) (width 1) (layer "F.Cu") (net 19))
 (segment (start -19.05 27.94) (end -18.415 28.575) (width 1) (layer "F.Cu") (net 19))
 (segment (start -16.51 24.13) (end -18.415 22.225) (width 1) (layer "F.Cu") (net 20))
 (segment (start -16.51 25.4) (end -16.51 24.13) (width 1) (layer "F.Cu") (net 20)))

